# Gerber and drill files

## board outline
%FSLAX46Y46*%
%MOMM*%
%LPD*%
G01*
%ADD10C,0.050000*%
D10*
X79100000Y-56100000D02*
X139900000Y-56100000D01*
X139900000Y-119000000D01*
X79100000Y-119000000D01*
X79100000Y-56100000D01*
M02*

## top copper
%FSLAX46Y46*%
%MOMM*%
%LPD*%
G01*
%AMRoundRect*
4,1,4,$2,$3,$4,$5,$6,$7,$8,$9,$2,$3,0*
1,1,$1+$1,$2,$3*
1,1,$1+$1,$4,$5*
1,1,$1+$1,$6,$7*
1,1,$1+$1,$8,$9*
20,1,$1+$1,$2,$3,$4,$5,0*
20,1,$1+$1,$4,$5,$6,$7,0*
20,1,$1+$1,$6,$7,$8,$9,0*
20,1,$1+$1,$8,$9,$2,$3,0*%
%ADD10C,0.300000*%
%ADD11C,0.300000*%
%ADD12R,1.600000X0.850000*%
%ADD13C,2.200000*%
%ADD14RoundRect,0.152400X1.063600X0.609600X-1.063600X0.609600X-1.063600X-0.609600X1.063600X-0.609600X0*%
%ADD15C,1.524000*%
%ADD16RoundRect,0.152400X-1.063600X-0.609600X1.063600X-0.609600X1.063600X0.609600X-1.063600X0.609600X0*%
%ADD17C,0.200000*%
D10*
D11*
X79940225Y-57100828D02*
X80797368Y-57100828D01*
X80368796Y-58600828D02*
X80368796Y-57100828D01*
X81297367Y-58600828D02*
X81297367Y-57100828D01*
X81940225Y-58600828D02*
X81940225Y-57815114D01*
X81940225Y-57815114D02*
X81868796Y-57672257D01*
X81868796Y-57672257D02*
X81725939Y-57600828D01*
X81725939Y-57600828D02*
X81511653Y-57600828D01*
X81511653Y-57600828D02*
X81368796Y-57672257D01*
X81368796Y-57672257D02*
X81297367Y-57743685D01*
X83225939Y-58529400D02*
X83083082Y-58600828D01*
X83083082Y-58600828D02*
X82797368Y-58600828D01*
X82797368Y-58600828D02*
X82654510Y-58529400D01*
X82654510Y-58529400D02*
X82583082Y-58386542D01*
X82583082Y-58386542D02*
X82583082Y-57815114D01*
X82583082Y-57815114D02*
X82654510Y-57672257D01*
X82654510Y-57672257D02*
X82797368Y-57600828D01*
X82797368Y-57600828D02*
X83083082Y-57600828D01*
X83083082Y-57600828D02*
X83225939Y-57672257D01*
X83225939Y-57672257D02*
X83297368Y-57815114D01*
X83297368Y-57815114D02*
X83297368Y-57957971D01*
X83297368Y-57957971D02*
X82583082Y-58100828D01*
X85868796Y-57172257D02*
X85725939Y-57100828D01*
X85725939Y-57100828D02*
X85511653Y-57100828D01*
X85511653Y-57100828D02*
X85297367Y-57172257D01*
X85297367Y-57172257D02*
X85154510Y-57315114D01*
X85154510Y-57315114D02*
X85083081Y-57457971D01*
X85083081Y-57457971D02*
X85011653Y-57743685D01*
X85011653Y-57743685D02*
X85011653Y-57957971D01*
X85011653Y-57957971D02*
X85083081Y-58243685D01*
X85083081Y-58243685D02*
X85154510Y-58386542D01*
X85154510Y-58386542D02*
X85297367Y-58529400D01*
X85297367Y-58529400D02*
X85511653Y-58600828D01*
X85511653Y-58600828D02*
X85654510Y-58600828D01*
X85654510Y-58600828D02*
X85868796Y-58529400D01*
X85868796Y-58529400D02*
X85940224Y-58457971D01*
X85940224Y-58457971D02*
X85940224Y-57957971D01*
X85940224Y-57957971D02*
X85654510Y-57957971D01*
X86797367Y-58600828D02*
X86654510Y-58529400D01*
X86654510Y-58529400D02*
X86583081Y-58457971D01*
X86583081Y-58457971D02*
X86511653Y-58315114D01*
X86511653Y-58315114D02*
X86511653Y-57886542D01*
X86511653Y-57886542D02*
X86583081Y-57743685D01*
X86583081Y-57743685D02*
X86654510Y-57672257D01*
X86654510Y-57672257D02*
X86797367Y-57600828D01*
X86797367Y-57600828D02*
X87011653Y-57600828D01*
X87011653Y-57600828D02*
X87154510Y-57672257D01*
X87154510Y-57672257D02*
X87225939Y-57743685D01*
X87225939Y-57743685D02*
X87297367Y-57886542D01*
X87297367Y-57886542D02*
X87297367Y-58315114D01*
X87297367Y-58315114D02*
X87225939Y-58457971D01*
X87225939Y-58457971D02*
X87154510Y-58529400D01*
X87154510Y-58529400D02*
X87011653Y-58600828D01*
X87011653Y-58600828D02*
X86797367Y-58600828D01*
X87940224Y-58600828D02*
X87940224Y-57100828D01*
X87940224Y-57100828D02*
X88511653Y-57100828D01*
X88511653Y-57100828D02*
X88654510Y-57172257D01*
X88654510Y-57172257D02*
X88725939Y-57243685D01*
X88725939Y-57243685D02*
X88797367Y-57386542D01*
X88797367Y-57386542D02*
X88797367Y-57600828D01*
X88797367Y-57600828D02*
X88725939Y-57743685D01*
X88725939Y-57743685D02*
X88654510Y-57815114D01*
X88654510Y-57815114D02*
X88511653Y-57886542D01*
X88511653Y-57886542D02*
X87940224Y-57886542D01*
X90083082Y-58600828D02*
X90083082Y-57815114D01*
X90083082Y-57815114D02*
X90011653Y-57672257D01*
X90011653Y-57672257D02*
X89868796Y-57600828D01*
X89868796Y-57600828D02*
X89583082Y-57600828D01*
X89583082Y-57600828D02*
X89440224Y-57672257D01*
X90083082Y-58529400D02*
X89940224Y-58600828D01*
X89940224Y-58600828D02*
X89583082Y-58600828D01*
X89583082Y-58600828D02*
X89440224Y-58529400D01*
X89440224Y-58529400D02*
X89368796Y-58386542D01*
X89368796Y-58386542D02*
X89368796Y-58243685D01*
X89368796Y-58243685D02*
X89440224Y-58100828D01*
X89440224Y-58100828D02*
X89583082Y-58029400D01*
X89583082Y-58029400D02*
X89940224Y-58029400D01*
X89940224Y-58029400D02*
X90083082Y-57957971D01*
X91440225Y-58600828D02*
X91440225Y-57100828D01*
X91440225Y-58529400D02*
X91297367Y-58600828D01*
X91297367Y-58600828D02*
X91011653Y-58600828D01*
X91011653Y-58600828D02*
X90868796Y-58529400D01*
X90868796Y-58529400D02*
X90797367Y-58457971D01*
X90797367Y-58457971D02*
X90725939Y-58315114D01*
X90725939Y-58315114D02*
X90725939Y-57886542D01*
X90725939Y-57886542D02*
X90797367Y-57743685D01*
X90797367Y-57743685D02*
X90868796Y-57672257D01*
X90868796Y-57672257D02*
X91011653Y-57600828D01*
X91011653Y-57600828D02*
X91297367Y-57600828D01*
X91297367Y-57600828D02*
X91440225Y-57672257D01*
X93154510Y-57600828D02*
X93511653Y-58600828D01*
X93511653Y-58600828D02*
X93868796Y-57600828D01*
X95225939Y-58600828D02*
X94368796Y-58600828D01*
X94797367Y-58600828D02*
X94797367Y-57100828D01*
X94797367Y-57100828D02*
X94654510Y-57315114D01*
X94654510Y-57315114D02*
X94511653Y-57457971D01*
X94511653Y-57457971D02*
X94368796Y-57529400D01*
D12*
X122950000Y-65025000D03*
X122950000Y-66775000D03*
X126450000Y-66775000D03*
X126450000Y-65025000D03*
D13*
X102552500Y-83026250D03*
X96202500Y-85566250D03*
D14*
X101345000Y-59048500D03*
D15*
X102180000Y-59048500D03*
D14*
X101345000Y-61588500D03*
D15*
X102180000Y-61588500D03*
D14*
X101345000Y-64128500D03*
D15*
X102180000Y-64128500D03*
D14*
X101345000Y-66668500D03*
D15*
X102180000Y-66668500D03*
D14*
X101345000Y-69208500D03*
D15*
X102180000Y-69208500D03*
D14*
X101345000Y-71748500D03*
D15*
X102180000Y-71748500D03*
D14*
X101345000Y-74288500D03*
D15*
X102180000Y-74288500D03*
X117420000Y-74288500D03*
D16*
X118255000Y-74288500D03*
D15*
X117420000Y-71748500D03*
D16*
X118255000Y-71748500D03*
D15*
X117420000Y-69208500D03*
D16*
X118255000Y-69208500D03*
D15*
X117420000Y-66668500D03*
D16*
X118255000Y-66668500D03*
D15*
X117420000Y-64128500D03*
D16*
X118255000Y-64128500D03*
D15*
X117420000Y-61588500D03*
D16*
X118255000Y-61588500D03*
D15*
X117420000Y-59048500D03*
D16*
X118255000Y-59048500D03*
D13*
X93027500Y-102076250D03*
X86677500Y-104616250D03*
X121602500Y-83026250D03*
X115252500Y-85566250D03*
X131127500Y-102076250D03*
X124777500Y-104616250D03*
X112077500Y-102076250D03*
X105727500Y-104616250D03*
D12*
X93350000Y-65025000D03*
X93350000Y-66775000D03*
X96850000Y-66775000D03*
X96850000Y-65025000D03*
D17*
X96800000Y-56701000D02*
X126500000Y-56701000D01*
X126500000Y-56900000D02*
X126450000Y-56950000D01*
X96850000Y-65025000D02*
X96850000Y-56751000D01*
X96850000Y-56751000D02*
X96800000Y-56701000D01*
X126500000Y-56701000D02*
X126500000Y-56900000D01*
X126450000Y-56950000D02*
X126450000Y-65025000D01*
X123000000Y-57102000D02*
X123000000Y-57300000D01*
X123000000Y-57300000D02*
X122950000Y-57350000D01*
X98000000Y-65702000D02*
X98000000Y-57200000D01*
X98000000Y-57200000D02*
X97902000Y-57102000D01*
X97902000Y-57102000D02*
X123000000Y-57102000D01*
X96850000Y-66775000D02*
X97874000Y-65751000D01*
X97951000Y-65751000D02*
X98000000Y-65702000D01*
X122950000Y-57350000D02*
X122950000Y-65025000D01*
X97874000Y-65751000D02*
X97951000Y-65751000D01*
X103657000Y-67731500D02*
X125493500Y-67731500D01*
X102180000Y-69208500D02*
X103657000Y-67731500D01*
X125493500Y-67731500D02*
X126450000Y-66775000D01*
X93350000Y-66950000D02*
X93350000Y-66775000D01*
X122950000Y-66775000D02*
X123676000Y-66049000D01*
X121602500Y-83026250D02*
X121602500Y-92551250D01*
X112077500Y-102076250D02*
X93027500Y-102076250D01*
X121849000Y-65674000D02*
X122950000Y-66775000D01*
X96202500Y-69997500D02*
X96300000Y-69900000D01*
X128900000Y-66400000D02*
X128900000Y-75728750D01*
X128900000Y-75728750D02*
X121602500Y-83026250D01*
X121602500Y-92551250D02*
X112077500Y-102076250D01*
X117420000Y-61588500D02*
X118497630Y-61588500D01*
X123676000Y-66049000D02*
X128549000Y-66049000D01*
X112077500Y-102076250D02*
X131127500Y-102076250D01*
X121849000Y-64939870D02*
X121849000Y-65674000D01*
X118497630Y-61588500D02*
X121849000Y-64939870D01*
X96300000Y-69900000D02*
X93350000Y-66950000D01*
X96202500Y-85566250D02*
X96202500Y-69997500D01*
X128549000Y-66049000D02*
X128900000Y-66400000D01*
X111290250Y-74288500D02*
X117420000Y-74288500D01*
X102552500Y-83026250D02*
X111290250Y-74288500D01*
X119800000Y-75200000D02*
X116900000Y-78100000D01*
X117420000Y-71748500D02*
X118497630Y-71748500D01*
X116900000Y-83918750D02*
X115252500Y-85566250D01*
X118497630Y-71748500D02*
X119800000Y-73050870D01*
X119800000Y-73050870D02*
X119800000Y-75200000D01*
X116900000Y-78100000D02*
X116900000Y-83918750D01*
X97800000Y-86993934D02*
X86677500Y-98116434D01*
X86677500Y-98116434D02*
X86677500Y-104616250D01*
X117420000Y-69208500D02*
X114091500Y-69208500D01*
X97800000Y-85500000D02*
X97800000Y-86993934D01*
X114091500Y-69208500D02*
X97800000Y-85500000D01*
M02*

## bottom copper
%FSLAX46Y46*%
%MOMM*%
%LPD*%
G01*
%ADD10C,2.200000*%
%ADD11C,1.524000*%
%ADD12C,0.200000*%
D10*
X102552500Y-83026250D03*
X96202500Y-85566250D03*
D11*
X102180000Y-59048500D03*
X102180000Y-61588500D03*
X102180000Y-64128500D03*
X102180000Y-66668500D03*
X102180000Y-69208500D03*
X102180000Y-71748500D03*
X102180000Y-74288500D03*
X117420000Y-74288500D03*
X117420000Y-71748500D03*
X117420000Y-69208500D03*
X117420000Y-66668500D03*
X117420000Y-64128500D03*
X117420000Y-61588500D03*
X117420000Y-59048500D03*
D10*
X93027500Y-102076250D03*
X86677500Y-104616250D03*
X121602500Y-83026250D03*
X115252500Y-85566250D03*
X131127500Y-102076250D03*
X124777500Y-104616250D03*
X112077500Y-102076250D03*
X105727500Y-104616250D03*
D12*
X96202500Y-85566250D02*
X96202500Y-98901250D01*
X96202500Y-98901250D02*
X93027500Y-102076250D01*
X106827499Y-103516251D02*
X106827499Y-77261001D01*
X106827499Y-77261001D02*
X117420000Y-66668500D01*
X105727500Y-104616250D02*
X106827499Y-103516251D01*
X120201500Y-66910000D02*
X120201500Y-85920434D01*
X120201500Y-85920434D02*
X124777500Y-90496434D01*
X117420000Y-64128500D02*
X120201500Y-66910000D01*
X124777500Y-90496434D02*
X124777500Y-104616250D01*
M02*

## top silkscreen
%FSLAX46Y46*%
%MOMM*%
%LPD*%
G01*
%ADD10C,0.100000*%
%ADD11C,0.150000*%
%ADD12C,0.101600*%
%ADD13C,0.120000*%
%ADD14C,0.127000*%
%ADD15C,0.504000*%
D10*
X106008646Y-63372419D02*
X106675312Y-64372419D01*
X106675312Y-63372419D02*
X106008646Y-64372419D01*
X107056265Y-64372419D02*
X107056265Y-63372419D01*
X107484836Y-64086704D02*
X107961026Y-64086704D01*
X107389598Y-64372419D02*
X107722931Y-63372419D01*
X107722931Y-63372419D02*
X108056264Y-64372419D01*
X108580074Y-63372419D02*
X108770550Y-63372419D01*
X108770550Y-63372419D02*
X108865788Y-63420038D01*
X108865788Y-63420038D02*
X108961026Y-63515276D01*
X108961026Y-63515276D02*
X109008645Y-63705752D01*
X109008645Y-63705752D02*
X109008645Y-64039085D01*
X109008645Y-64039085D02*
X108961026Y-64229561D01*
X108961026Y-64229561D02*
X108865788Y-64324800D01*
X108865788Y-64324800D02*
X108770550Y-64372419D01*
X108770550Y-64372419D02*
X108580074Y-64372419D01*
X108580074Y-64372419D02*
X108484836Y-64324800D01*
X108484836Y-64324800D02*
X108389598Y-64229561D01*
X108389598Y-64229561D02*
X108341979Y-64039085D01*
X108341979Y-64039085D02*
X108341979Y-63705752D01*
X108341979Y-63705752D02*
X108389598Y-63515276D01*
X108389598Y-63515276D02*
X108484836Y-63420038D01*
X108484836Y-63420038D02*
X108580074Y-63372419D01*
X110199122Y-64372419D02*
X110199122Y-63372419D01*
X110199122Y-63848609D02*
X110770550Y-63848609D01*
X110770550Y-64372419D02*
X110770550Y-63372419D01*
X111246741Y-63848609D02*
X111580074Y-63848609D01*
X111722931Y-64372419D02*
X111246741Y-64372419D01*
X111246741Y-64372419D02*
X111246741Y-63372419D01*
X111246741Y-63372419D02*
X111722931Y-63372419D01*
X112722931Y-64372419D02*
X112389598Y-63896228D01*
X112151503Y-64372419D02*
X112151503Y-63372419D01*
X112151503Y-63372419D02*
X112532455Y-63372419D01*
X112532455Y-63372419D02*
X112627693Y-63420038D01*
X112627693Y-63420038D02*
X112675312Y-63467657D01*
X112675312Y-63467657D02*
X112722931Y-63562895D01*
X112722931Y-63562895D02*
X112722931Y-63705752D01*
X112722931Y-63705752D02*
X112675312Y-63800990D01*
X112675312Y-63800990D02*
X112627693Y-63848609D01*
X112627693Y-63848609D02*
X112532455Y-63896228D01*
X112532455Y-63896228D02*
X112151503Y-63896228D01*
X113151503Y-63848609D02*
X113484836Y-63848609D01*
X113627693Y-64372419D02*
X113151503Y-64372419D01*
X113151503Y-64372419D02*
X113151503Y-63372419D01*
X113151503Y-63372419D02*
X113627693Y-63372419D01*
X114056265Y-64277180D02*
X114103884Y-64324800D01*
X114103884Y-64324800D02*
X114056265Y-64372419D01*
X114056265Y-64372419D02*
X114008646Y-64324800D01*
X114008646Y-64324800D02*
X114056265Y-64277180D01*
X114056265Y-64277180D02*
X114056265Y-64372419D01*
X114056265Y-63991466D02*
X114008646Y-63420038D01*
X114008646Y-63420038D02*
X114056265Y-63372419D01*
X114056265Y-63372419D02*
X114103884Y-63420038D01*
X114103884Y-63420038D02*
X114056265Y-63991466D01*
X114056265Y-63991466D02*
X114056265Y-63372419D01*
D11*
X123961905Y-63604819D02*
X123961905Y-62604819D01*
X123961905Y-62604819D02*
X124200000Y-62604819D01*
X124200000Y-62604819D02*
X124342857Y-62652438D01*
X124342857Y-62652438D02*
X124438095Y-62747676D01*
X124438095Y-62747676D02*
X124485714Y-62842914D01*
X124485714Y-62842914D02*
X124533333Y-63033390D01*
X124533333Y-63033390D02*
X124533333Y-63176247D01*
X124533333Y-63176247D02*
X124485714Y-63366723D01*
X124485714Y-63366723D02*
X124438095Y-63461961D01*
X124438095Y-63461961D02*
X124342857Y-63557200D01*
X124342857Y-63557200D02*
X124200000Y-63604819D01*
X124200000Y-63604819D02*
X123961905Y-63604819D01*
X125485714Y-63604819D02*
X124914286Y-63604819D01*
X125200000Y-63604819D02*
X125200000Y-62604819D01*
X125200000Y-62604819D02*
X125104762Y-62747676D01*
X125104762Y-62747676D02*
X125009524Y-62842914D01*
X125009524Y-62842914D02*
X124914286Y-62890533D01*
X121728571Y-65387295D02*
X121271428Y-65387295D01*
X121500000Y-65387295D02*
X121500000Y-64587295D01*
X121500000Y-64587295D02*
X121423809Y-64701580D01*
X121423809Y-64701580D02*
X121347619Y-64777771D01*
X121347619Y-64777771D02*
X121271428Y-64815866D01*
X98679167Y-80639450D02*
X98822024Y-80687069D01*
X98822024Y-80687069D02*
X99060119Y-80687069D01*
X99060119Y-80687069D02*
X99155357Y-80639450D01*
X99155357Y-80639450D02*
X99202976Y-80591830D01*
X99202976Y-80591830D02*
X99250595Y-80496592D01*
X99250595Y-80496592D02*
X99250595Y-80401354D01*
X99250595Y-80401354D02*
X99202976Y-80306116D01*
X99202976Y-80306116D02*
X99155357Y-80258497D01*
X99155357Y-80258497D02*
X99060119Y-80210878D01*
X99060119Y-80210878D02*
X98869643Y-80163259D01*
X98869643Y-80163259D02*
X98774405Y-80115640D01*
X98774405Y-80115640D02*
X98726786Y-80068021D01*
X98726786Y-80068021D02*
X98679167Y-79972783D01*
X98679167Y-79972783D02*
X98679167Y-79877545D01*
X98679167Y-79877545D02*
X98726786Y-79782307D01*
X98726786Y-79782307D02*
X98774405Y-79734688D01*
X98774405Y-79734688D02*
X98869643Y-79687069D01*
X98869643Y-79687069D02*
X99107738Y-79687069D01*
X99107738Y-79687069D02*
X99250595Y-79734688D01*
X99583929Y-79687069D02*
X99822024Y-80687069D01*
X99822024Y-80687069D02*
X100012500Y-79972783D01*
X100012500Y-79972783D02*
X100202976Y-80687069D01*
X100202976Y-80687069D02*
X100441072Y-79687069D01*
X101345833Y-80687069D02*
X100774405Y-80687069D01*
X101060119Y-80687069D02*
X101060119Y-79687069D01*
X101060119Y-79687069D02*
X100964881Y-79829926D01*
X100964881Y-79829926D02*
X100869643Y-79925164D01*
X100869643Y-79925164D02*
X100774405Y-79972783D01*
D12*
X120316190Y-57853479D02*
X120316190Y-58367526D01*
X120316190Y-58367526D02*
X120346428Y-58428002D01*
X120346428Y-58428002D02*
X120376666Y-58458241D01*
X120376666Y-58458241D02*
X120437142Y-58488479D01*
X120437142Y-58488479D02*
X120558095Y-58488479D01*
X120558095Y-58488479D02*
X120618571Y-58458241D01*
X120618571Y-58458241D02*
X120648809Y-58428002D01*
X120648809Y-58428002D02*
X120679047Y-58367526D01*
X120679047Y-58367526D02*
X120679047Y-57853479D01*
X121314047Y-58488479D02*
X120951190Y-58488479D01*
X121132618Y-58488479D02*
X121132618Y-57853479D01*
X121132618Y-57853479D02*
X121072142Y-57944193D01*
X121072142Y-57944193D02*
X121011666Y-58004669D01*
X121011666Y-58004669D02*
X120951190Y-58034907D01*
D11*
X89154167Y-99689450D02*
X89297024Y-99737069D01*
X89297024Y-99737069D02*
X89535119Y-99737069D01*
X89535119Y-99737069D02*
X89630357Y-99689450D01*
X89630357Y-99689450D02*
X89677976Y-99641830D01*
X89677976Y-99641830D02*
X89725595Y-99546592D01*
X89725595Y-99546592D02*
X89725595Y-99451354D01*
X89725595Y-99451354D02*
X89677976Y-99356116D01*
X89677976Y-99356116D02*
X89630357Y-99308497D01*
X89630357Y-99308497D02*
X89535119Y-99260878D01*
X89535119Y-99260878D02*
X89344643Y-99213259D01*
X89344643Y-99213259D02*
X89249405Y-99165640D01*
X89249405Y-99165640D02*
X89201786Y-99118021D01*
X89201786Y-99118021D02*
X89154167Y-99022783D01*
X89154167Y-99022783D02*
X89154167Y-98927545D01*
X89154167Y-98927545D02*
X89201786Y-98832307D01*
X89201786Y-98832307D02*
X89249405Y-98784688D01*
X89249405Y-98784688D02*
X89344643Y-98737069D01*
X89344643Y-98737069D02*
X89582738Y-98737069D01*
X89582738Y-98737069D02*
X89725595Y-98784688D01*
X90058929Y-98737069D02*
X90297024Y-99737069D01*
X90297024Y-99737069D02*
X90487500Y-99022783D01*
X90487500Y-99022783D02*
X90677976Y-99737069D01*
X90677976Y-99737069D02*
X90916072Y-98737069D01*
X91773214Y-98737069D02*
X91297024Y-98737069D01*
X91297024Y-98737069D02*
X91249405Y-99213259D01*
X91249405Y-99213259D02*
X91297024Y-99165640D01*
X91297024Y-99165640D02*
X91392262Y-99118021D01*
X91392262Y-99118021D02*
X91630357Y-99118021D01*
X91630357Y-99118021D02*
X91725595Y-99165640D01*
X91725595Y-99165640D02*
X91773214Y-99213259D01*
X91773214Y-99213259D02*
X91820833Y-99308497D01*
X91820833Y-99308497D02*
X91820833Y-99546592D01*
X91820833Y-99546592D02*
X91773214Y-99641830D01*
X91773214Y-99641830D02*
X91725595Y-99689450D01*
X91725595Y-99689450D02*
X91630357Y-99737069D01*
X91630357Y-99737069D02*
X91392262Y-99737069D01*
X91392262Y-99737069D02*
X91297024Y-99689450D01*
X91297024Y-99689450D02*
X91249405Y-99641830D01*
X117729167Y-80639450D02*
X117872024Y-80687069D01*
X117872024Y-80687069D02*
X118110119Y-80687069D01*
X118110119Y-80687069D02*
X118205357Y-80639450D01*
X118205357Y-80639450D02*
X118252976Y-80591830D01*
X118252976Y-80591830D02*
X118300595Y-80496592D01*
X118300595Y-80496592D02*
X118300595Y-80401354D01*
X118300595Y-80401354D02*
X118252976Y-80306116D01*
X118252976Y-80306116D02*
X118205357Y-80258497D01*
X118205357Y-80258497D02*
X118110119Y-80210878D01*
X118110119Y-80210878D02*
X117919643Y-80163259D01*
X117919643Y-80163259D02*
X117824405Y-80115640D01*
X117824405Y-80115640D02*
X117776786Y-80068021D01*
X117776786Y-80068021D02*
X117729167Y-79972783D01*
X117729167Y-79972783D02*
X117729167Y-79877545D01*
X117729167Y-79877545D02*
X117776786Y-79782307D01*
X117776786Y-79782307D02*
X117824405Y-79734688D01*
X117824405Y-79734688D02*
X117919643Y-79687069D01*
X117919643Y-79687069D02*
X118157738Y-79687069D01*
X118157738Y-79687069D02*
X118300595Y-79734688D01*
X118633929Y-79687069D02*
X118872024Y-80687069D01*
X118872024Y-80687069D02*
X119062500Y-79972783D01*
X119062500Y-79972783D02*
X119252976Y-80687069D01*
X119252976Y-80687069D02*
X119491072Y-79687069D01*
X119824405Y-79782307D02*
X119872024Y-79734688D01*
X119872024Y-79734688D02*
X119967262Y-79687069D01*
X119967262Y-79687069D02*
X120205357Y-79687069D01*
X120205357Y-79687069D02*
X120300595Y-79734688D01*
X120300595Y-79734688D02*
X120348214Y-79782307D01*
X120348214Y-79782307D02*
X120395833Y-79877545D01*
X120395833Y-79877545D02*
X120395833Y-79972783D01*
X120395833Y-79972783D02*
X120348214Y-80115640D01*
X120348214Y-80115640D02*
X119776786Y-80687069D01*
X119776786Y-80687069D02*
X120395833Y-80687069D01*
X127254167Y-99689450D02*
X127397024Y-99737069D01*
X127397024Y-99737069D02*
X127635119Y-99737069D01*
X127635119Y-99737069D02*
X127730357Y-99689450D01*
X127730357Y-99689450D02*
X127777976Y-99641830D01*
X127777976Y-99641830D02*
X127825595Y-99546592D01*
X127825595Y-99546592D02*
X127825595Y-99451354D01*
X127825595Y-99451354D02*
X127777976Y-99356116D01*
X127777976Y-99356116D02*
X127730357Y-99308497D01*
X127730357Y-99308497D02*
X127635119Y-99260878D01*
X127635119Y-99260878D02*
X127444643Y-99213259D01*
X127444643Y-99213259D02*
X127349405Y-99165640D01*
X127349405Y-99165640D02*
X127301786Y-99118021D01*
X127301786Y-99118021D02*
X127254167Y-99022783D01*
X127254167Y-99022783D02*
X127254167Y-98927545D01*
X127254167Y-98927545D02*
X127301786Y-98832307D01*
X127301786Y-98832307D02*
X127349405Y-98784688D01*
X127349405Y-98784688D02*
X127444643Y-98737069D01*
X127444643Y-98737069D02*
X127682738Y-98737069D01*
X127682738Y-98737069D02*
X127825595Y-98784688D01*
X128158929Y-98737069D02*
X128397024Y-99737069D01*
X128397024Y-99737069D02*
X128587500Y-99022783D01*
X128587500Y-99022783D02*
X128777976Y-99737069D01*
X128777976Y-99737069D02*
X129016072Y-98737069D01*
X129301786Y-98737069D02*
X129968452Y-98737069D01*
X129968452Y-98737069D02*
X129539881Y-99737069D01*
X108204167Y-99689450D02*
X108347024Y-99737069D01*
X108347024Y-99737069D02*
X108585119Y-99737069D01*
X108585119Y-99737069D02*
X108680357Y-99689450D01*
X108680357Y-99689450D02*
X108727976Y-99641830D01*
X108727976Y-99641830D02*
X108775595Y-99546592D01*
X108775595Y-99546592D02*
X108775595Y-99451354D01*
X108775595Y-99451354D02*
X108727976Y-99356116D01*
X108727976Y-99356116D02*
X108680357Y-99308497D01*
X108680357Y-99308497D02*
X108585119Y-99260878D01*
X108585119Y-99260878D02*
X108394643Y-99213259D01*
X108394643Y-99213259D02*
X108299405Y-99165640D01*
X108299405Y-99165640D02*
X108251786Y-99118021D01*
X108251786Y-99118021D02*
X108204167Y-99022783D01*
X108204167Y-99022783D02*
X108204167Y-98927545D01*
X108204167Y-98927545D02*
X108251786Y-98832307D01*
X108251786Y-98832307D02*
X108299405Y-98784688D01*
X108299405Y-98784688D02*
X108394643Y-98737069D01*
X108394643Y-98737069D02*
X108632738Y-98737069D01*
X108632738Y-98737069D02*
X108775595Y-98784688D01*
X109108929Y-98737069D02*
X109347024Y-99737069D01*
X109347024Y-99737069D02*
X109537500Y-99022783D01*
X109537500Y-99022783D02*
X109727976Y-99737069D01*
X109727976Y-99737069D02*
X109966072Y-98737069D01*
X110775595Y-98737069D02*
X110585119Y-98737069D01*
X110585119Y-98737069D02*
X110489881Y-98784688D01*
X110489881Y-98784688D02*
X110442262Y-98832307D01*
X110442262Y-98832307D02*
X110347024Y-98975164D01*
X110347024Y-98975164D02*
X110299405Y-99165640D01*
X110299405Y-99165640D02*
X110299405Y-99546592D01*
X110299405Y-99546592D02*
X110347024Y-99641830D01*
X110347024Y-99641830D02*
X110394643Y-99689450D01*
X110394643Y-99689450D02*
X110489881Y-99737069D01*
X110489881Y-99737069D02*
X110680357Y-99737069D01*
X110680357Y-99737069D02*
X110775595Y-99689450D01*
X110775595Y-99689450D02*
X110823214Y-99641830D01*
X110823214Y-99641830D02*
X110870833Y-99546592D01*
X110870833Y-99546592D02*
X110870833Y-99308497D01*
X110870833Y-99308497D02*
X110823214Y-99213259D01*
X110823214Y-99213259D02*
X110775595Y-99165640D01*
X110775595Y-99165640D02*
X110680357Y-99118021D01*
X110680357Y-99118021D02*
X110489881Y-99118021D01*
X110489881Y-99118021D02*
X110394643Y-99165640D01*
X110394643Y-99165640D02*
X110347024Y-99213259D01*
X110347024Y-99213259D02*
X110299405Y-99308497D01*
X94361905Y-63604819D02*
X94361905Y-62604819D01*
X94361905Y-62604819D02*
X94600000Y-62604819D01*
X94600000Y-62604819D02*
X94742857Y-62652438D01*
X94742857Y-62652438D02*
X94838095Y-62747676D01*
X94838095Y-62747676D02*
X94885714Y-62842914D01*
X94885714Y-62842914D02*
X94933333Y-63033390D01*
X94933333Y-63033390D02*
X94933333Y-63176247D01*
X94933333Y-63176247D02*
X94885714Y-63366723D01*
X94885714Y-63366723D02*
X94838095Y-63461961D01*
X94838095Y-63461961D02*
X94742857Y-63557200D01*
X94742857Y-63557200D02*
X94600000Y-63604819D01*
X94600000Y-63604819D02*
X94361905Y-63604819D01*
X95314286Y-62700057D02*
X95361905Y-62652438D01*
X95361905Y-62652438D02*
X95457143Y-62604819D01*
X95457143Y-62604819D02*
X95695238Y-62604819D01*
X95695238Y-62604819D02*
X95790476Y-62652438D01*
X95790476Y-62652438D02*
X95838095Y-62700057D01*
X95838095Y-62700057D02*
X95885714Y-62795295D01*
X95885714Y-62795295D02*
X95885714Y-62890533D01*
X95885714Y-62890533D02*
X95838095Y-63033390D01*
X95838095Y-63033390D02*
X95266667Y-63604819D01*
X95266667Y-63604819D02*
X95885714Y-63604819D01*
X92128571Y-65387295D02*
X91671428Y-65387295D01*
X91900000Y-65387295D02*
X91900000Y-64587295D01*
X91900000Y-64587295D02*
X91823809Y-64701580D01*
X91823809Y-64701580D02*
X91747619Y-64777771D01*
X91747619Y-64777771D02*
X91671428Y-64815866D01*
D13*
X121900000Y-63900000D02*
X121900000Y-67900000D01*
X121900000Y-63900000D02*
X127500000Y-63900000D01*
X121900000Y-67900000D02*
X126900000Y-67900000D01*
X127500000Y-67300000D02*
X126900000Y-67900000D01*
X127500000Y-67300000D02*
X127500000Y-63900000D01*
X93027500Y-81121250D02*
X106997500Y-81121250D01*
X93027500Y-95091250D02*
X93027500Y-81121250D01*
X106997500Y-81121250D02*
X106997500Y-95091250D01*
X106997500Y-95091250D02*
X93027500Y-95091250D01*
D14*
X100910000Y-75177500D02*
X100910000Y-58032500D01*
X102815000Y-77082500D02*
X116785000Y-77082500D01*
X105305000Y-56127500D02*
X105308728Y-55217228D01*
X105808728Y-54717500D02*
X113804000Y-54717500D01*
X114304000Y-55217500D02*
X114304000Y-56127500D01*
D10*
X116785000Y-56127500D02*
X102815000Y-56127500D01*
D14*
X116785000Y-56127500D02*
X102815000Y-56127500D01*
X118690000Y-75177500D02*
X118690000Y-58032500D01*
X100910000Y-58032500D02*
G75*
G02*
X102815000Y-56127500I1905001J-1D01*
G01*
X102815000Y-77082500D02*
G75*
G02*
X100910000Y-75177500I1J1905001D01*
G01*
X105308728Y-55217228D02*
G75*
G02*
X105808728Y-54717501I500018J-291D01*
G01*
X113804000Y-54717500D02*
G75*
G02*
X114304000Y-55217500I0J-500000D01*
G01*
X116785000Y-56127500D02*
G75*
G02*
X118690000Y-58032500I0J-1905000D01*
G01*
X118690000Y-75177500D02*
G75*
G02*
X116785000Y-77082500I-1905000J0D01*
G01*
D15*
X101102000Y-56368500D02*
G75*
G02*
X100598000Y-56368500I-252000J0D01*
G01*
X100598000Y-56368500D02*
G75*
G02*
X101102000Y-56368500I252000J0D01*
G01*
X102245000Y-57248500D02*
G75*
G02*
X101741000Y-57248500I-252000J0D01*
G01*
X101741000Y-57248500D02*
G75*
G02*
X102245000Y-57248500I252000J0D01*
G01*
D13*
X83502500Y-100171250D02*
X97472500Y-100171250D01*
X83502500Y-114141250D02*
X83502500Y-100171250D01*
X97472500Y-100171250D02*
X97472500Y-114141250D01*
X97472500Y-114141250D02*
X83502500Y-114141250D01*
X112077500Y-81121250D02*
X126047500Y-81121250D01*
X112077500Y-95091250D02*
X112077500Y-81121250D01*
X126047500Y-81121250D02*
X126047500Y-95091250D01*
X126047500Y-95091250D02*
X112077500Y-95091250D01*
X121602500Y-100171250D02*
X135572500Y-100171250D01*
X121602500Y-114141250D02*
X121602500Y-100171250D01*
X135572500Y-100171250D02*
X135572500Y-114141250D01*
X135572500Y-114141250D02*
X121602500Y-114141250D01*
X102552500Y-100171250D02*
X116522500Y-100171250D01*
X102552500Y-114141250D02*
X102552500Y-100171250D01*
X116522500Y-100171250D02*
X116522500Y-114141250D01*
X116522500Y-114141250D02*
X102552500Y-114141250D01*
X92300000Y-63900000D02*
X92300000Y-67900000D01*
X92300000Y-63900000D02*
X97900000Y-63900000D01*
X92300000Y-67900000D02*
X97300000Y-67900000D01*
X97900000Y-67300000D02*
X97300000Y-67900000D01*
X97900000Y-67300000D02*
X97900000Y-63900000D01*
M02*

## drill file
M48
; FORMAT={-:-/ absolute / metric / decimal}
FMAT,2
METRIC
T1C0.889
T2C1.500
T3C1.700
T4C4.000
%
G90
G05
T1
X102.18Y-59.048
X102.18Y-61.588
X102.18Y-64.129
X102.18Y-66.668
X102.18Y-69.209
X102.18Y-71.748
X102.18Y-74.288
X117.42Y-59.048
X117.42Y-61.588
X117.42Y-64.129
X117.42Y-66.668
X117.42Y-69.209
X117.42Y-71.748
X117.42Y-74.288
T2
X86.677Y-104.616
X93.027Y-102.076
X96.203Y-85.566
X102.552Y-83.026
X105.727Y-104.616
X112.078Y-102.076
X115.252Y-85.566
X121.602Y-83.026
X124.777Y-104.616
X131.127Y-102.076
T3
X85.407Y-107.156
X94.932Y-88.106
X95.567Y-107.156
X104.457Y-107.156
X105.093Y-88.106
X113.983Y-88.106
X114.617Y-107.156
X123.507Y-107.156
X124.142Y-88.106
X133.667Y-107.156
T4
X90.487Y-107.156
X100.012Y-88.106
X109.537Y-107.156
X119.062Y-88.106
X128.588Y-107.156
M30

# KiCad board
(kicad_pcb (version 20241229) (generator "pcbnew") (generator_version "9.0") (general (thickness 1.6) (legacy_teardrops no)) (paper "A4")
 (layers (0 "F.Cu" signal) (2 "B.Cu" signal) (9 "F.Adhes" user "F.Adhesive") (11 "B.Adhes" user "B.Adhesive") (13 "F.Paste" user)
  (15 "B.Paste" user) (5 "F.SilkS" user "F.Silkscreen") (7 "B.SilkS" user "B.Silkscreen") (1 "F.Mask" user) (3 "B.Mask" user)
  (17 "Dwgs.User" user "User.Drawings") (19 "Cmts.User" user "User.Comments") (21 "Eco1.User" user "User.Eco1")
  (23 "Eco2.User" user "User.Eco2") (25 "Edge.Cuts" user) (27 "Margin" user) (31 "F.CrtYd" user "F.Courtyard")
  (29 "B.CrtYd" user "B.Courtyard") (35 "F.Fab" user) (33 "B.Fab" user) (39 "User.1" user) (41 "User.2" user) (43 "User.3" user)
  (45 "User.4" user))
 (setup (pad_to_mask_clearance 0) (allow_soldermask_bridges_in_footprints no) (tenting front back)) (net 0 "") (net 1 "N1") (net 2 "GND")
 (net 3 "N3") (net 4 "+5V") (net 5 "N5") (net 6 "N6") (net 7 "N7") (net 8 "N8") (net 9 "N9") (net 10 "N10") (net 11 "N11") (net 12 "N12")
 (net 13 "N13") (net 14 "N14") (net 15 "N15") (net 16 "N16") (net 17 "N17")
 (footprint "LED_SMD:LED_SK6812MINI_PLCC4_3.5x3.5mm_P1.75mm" (layer "F.Cu") (at 124.7 65.9)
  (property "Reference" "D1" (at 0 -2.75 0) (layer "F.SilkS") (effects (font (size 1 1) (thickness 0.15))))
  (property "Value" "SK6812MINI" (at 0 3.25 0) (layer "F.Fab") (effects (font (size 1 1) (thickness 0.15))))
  (fp_line (start -2.8 -2) (end -2.8 2) (stroke (width 0.12) (type default)) (layer "F.SilkS"))
  (fp_line (start -2.8 -2) (end 2.8 -2) (stroke (width 0.12) (type solid)) (layer "F.SilkS"))
  (fp_line (start -2.8 2) (end 2.2 2) (stroke (width 0.12) (type solid)) (layer "F.SilkS"))
  (fp_line (start 2.8 1.4) (end 2.2 2) (stroke (width 0.12) (type default)) (layer "F.SilkS"))
  (fp_line (start 2.8 1.4) (end 2.8 -2) (stroke (width 0.12) (type solid)) (layer "F.SilkS"))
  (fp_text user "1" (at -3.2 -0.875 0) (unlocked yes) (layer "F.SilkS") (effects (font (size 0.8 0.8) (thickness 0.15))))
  (pad "1" smd rect (at -1.75 -0.875) (size 1.6 0.85) (layers "F.Cu" "F.Mask" "F.Paste") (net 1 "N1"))
  (pad "2" smd rect (at -1.75 0.875) (size 1.6 0.85) (layers "F.Cu" "F.Mask" "F.Paste") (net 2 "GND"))
  (pad "3" smd rect (at 1.75 0.875) (size 1.6 0.85) (layers "F.Cu" "F.Mask" "F.Paste") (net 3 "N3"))
  (pad "4" smd rect (at 1.75 -0.875) (size 1.6 0.85) (layers "F.Cu" "F.Mask" "F.Paste") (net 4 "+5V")))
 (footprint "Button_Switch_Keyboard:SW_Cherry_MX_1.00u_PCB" (layer "F.Cu") (at 102.5525 83.02625)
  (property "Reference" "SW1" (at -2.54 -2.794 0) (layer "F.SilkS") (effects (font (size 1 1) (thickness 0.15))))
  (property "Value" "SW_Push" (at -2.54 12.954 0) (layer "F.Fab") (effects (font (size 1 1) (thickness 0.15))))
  (fp_line (start -9.525 -1.905) (end 4.445 -1.905) (stroke (width 0.12) (type solid)) (layer "F.SilkS"))
  (fp_line (start -9.525 12.065) (end -9.525 -1.905) (stroke (width 0.12) (type solid)) (layer "F.SilkS"))
  (fp_line (start 4.445 -1.905) (end 4.445 12.065) (stroke (width 0.12) (type solid)) (layer "F.SilkS"))
  (fp_line (start 4.445 12.065) (end -9.525 12.065) (stroke (width 0.12) (type solid)) (layer "F.SilkS"))
  (pad "" np_thru_hole circle (at -7.62 5.08) (size 1.7 1.7) (drill 1.7) (layers "*.Cu" "*.Mask"))
  (pad "" np_thru_hole circle (at -2.54 5.08) (size 4 4) (drill 4) (layers "*.Cu" "*.Mask"))
  (pad "" np_thru_hole circle (at 2.54 5.08) (size 1.7 1.7) (drill 1.7) (layers "*.Cu" "*.Mask"))
  (pad "1" thru_hole circle (at 0 0) (size 2.2 2.2) (drill 1.5) (layers "*.Cu" "*.Mask") (remove_unused_layers no) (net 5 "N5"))
  (pad "2" thru_hole circle (at -6.35 2.54) (size 2.2 2.2) (drill 1.5) (layers "*.Cu" "*.Mask") (remove_unused_layers no) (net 2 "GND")))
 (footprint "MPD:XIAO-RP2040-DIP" (layer "F.Cu") (at 109.8 66.6685)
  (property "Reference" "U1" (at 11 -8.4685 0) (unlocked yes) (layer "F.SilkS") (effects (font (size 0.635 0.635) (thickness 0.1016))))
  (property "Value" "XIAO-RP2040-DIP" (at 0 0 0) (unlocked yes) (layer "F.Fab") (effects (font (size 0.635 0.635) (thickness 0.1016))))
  (fp_line (start -8.89 8.509) (end -8.89 -8.636) (stroke (width 0.127) (type solid)) (layer "F.SilkS"))
  (fp_line (start -6.985 10.414) (end 6.985 10.414) (stroke (width 0.127) (type solid)) (layer "F.SilkS"))
  (fp_line (start -4.495 -10.541) (end -4.491272 -11.451272) (stroke (width 0.127) (type solid)) (layer "F.SilkS"))
  (fp_line (start -3.991272 -11.951) (end 4.004 -11.951) (stroke (width 0.127) (type solid)) (layer "F.SilkS"))
  (fp_line (start 4.504 -11.451) (end 4.504 -10.541) (stroke (width 0.127) (type solid)) (layer "F.SilkS"))
  (fp_line (start 6.985 -10.541) (end -6.985 -10.541) (stroke (width 0.1) (type solid)) (layer "F.SilkS"))
  (fp_line (start 6.985 -10.541) (end -6.985 -10.541) (stroke (width 0.127) (type solid)) (layer "F.SilkS"))
  (fp_line (start 8.89 8.509) (end 8.89 -8.636) (stroke (width 0.127) (type solid)) (layer "F.SilkS"))
  (fp_arc (start -8.89 -8.636) (mid -8.332038 -9.983038) (end -6.985 -10.541) (stroke (width 0.127) (type solid)) (layer "F.SilkS"))
  (fp_arc (start -6.985 10.414) (mid -8.332038 9.856038) (end -8.89 8.509) (stroke (width 0.127) (type solid)) (layer "F.SilkS"))
  (fp_arc (start -4.491272 -11.451272) (mid -4.344728 -11.80464) (end -3.991272 -11.951) (stroke (width 0.127) (type default))
   (layer "F.SilkS"))
  (fp_arc (start 4.004 -11.951) (mid 4.357553 -11.804553) (end 4.504 -11.451) (stroke (width 0.127) (type default)) (layer "F.SilkS"))
  (fp_arc (start 6.985 -10.541) (mid 8.332038 -9.983038) (end 8.89 -8.636) (stroke (width 0.127) (type solid)) (layer "F.SilkS"))
  (fp_arc (start 8.89 8.509) (mid 8.332038 9.856038) (end 6.985 10.414) (stroke (width 0.127) (type solid)) (layer "F.SilkS"))
  (fp_circle (center -8.95 -10.3) (end -8.95 -10.554) (stroke (width 0.5) (type solid)) (fill yes) (layer "F.SilkS"))
  (fp_circle (center -7.807 -9.42) (end -7.807 -9.674) (stroke (width 0.5) (type solid)) (fill yes) (layer "F.SilkS"))
  (pad "1" smd roundrect (at -8.455 -7.62 180) (size 2.432 1.524) (layers "F.Cu" "F.Mask") (roundrect_rratio 0.1) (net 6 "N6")
   (thermal_bridge_angle 45))
  (pad "1" thru_hole circle (at -7.62 -7.62 180) (size 1.524 1.524) (drill 0.889) (layers "*.Cu" "*.Mask") (remove_unused_layers no)
   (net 6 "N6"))
  (pad "2" smd roundrect (at -8.455 -5.08 180) (size 2.432 1.524) (layers "F.Cu" "F.Mask") (roundrect_rratio 0.1) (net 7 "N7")
   (thermal_bridge_angle 45))
  (pad "2" thru_hole circle (at -7.62 -5.08 180) (size 1.524 1.524) (drill 0.889) (layers "*.Cu" "*.Mask") (remove_unused_layers no)
   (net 7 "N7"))
  (pad "3" smd roundrect (at -8.455 -2.54 180) (size 2.432 1.524) (layers "F.Cu" "F.Mask") (roundrect_rratio 0.1) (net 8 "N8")
   (thermal_bridge_angle 45))
  (pad "3" thru_hole circle (at -7.62 -2.54 180) (size 1.524 1.524) (drill 0.889) (layers "*.Cu" "*.Mask") (remove_unused_layers no)
   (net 8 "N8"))
  (pad "4" smd roundrect (at -8.455 0 180) (size 2.432 1.524) (layers "F.Cu" "F.Mask") (roundrect_rratio 0.1) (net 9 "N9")
   (thermal_bridge_angle 45))
  (pad "4" thru_hole circle (at -7.62 0 180) (size 1.524 1.524) (drill 0.889) (layers "*.Cu" "*.Mask") (remove_unused_layers no)
   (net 9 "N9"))
  (pad "5" smd roundrect (at -8.455 2.54 180) (size 2.432 1.524) (layers "F.Cu" "F.Mask") (roundrect_rratio 0.1) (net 3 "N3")
   (thermal_bridge_angle 45))
  (pad "5" thru_hole circle (at -7.62 2.54 180) (size 1.524 1.524) (drill 0.889) (layers "*.Cu" "*.Mask") (remove_unused_layers no)
   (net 3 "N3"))
  (pad "6" smd roundrect (at -8.455 5.08 180) (size 2.432 1.524) (layers "F.Cu" "F.Mask") (roundrect_rratio 0.1) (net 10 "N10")
   (thermal_bridge_angle 45))
  (pad "6" thru_hole circle (at -7.62 5.08 180) (size 1.524 1.524) (drill 0.889) (layers "*.Cu" "*.Mask") (remove_unused_layers no)
   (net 10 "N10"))
  (pad "7" smd roundrect (at -8.455 7.62 180) (size 2.432 1.524) (layers "F.Cu" "F.Mask") (roundrect_rratio 0.1) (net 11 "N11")
   (thermal_bridge_angle 45))
  (pad "7" thru_hole circle (at -7.62 7.62 180) (size 1.524 1.524) (drill 0.889) (layers "*.Cu" "*.Mask") (remove_unused_layers no)
   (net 11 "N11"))
  (pad "8" thru_hole circle (at 7.62 7.62) (size 1.524 1.524) (drill 0.889) (layers "*.Cu" "*.Mask") (remove_unused_layers no) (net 5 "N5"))
  (pad "8" smd roundrect (at 8.455 7.62) (size 2.432 1.524) (layers "F.Cu" "F.Mask") (roundrect_rratio 0.1) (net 5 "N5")
   (thermal_bridge_angle 45))
  (pad "9" thru_hole circle (at 7.62 5.08) (size 1.524 1.524) (drill 0.889) (layers "*.Cu" "*.Mask") (remove_unused_layers no)
   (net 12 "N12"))
  (pad "9" smd roundrect (at 8.455 5.08) (size 2.432 1.524) (layers "F.Cu" "F.Mask") (roundrect_rratio 0.1) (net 12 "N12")
   (thermal_bridge_angle 45))
  (pad "10" thru_hole circle (at 7.62 2.54) (size 1.524 1.524) (drill 0.889) (layers "*.Cu" "*.Mask") (remove_unused_layers no)
   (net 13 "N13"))
  (pad "10" smd roundrect (at 8.455 2.54) (size 2.432 1.524) (layers "F.Cu" "F.Mask") (roundrect_rratio 0.1) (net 13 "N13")
   (thermal_bridge_angle 45))
  (pad "11" thru_hole circle (at 7.62 0) (size 1.524 1.524) (drill 0.889) (layers "*.Cu" "*.Mask") (remove_unused_layers no) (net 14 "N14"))
  (pad "11" smd roundrect (at 8.455 0) (size 2.432 1.524) (layers "F.Cu" "F.Mask") (roundrect_rratio 0.1) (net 14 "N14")
   (thermal_bridge_angle 45))
  (pad "12" thru_hole circle (at 7.62 -2.54) (size 1.524 1.524) (drill 0.889) (layers "*.Cu" "*.Mask") (remove_unused_layers no)
   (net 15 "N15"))
  (pad "12" smd roundrect (at 8.455 -2.54) (size 2.432 1.524) (layers "F.Cu" "F.Mask") (roundrect_rratio 0.1) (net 15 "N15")
   (thermal_bridge_angle 45))
  (pad "13" thru_hole circle (at 7.62 -5.08) (size 1.524 1.524) (drill 0.889) (layers "*.Cu" "*.Mask") (remove_unused_layers no)
   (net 2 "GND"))
  (pad "13" smd roundrect (at 8.455 -5.08) (size 2.432 1.524) (layers "F.Cu" "F.Mask") (roundrect_rratio 0.1) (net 2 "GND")
   (thermal_bridge_angle 45))
  (pad "14" thru_hole circle (at 7.62 -7.62) (size 1.524 1.524) (drill 0.889) (layers "*.Cu" "*.Mask") (remove_unused_layers no)
   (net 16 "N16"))
  (pad "14" smd roundrect (at 8.455 -7.62) (size 2.432 1.524) (layers "F.Cu" "F.Mask") (roundrect_rratio 0.1) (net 16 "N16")
   (thermal_bridge_angle 45)))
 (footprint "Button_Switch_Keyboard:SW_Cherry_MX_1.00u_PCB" (layer "F.Cu") (at 93.0275 102.07625)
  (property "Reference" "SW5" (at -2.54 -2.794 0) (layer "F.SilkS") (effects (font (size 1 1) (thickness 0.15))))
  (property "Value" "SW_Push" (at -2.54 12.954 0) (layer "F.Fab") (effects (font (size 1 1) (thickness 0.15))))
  (fp_line (start -9.525 -1.905) (end 4.445 -1.905) (stroke (width 0.12) (type solid)) (layer "F.SilkS"))
  (fp_line (start -9.525 12.065) (end -9.525 -1.905) (stroke (width 0.12) (type solid)) (layer "F.SilkS"))
  (fp_line (start 4.445 -1.905) (end 4.445 12.065) (stroke (width 0.12) (type solid)) (layer "F.SilkS"))
  (fp_line (start 4.445 12.065) (end -9.525 12.065) (stroke (width 0.12) (type solid)) (layer "F.SilkS"))
  (pad "" np_thru_hole circle (at -7.62 5.08) (size 1.7 1.7) (drill 1.7) (layers "*.Cu" "*.Mask"))
  (pad "" np_thru_hole circle (at -2.54 5.08) (size 4 4) (drill 4) (layers "*.Cu" "*.Mask"))
  (pad "" np_thru_hole circle (at 2.54 5.08) (size 1.7 1.7) (drill 1.7) (layers "*.Cu" "*.Mask"))
  (pad "1" thru_hole circle (at 0 0) (size 2.2 2.2) (drill 1.5) (layers "*.Cu" "*.Mask") (remove_unused_layers no) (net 2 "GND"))
  (pad "2" thru_hole circle (at -6.35 2.54) (size 2.2 2.2) (drill 1.5) (layers "*.Cu" "*.Mask") (remove_unused_layers no) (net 13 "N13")))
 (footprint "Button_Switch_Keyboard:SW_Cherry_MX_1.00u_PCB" (layer "F.Cu") (at 121.6025 83.02625)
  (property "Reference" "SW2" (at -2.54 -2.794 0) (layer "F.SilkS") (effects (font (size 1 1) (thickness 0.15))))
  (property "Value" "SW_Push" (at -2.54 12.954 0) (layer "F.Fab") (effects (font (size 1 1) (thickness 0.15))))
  (fp_line (start -9.525 -1.905) (end 4.445 -1.905) (stroke (width 0.12) (type solid)) (layer "F.SilkS"))
  (fp_line (start -9.525 12.065) (end -9.525 -1.905) (stroke (width 0.12) (type solid)) (layer "F.SilkS"))
  (fp_line (start 4.445 -1.905) (end 4.445 12.065) (stroke (width 0.12) (type solid)) (layer "F.SilkS"))
  (fp_line (start 4.445 12.065) (end -9.525 12.065) (stroke (width 0.12) (type solid)) (layer "F.SilkS"))
  (pad "" np_thru_hole circle (at -7.62 5.08) (size 1.7 1.7) (drill 1.7) (layers "*.Cu" "*.Mask"))
  (pad "" np_thru_hole circle (at -2.54 5.08) (size 4 4) (drill 4) (layers "*.Cu" "*.Mask"))
  (pad "" np_thru_hole circle (at 2.54 5.08) (size 1.7 1.7) (drill 1.7) (layers "*.Cu" "*.Mask"))
  (pad "1" thru_hole circle (at 0 0) (size 2.2 2.2) (drill 1.5) (layers "*.Cu" "*.Mask") (remove_unused_layers no) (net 2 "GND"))
  (pad "2" thru_hole circle (at -6.35 2.54) (size 2.2 2.2) (drill 1.5) (layers "*.Cu" "*.Mask") (remove_unused_layers no) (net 12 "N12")))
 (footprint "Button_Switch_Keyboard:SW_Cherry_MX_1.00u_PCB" (layer "F.Cu") (at 131.1275 102.07625)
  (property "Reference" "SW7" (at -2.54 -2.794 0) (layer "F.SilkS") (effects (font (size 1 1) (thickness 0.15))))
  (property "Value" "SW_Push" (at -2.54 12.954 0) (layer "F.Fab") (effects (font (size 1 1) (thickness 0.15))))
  (fp_line (start -9.525 -1.905) (end 4.445 -1.905) (stroke (width 0.12) (type solid)) (layer "F.SilkS"))
  (fp_line (start -9.525 12.065) (end -9.525 -1.905) (stroke (width 0.12) (type solid)) (layer "F.SilkS"))
  (fp_line (start 4.445 -1.905) (end 4.445 12.065) (stroke (width 0.12) (type solid)) (layer "F.SilkS"))
  (fp_line (start 4.445 12.065) (end -9.525 12.065) (stroke (width 0.12) (type solid)) (layer "F.SilkS"))
  (pad "" np_thru_hole circle (at -7.62 5.08) (size 1.7 1.7) (drill 1.7) (layers "*.Cu" "*.Mask"))
  (pad "" np_thru_hole circle (at -2.54 5.08) (size 4 4) (drill 4) (layers "*.Cu" "*.Mask"))
  (pad "" np_thru_hole circle (at 2.54 5.08) (size 1.7 1.7) (drill 1.7) (layers "*.Cu" "*.Mask"))
  (pad "1" thru_hole circle (at 0 0) (size 2.2 2.2) (drill 1.5) (layers "*.Cu" "*.Mask") (remove_unused_layers no) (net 2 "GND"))
  (pad "2" thru_hole circle (at -6.35 2.54) (size 2.2 2.2) (drill 1.5) (layers "*.Cu" "*.Mask") (remove_unused_layers no) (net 15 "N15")))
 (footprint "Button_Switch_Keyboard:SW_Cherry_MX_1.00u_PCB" (layer "F.Cu") (at 112.0775 102.07625)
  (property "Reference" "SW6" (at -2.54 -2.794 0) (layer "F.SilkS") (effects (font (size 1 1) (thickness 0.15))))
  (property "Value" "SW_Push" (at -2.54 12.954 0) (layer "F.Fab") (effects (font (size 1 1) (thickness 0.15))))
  (fp_line (start -9.525 -1.905) (end 4.445 -1.905) (stroke (width 0.12) (type solid)) (layer "F.SilkS"))
  (fp_line (start -9.525 12.065) (end -9.525 -1.905) (stroke (width 0.12) (type solid)) (layer "F.SilkS"))
  (fp_line (start 4.445 -1.905) (end 4.445 12.065) (stroke (width 0.12) (type solid)) (layer "F.SilkS"))
  (fp_line (start 4.445 12.065) (end -9.525 12.065) (stroke (width 0.12) (type solid)) (layer "F.SilkS"))
  (pad "" np_thru_hole circle (at -7.62 5.08) (size 1.7 1.7) (drill 1.7) (layers "*.Cu" "*.Mask"))
  (pad "" np_thru_hole circle (at -2.54 5.08) (size 4 4) (drill 4) (layers "*.Cu" "*.Mask"))
  (pad "" np_thru_hole circle (at 2.54 5.08) (size 1.7 1.7) (drill 1.7) (layers "*.Cu" "*.Mask"))
  (pad "1" thru_hole circle (at 0 0) (size 2.2 2.2) (drill 1.5) (layers "*.Cu" "*.Mask") (remove_unused_layers no) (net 2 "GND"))
  (pad "2" thru_hole circle (at -6.35 2.54) (size 2.2 2.2) (drill 1.5) (layers "*.Cu" "*.Mask") (remove_unused_layers no) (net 14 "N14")))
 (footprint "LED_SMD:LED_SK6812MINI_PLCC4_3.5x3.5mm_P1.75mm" (layer "F.Cu") (at 95.1 65.9)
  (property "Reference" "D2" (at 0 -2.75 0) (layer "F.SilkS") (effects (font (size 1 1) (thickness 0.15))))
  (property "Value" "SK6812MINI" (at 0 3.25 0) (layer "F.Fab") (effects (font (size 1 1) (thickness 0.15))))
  (fp_line (start -2.8 -2) (end -2.8 2) (stroke (width 0.12) (type default)) (layer "F.SilkS"))
  (fp_line (start -2.8 -2) (end 2.8 -2) (stroke (width 0.12) (type solid)) (layer "F.SilkS"))
  (fp_line (start -2.8 2) (end 2.2 2) (stroke (width 0.12) (type solid)) (layer "F.SilkS"))
  (fp_line (start 2.8 1.4) (end 2.2 2) (stroke (width 0.12) (type default)) (layer "F.SilkS"))
  (fp_line (start 2.8 1.4) (end 2.8 -2) (stroke (width 0.12) (type solid)) (layer "F.SilkS"))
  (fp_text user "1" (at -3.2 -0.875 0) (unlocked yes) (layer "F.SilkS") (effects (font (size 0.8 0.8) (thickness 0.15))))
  (pad "1" smd rect (at -1.75 -0.875) (size 1.6 0.85) (layers "F.Cu" "F.Mask" "F.Paste") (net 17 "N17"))
  (pad "2" smd rect (at -1.75 0.875) (size 1.6 0.85) (layers "F.Cu" "F.Mask" "F.Paste") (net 2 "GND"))
  (pad "3" smd rect (at 1.75 0.875) (size 1.6 0.85) (layers "F.Cu" "F.Mask" "F.Paste") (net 1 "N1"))
  (pad "4" smd rect (at 1.75 -0.875) (size 1.6 0.85) (layers "F.Cu" "F.Mask" "F.Paste") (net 4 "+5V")))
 (gr_rect (start 79.1 56.1) (end 139.9 119) (stroke (width 0.05) (type default)) (fill no) (layer "Edge.Cuts"))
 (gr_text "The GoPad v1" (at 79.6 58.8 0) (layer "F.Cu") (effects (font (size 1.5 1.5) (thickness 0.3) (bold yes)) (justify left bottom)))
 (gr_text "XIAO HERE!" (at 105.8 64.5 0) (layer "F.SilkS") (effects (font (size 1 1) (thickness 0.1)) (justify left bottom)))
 (segment (start 96.8 56.701) (end 126.5 56.701) (width 0.2) (layer "F.Cu") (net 4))
 (segment (start 126.5 56.9) (end 126.45 56.95) (width 0.2) (layer "F.Cu") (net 4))
 (segment (start 96.85 65.025) (end 96.85 56.751) (width 0.2) (layer "F.Cu") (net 4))
 (segment (start 96.85 56.751) (end 96.8 56.701) (width 0.2) (layer "F.Cu") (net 4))
 (segment (start 126.5 56.701) (end 126.5 56.9) (width 0.2) (layer "F.Cu") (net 4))
 (segment (start 126.45 56.95) (end 126.45 65.025) (width 0.2) (layer "F.Cu") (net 4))
 (segment (start 123 57.102) (end 123 57.3) (width 0.2) (layer "F.Cu") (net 1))
 (segment (start 123 57.3) (end 122.95 57.35) (width 0.2) (layer "F.Cu") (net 1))
 (segment (start 98 65.702) (end 98 57.2) (width 0.2) (layer "F.Cu") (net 1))
 (segment (start 98 57.2) (end 97.902 57.102) (width 0.2) (layer "F.Cu") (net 1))
 (segment (start 97.902 57.102) (end 123 57.102) (width 0.2) (layer "F.Cu") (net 1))
 (segment (start 96.85 66.775) (end 97.874 65.751) (width 0.2) (layer "F.Cu") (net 1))
 (segment (start 97.951 65.751) (end 98 65.702) (width 0.2) (layer "F.Cu") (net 1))
 (segment (start 122.95 57.35) (end 122.95 65.025) (width 0.2) (layer "F.Cu") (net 1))
 (segment (start 97.874 65.751) (end 97.951 65.751) (width 0.2) (layer "F.Cu") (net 1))
 (segment (start 103.657 67.7315) (end 125.4935 67.7315) (width 0.2) (layer "F.Cu") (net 3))
 (segment (start 102.18 69.2085) (end 103.657 67.7315) (width 0.2) (layer "F.Cu") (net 3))
 (segment (start 125.4935 67.7315) (end 126.45 66.775) (width 0.2) (layer "F.Cu") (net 3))
 (segment (start 93.35 66.95) (end 93.35 66.775) (width 0.2) (layer "F.Cu") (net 2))
 (segment (start 122.95 66.775) (end 123.676 66.049) (width 0.2) (layer "F.Cu") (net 2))
 (segment (start 121.6025 83.02625) (end 121.6025 92.55125) (width 0.2) (layer "F.Cu") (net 2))
 (segment (start 112.0775 102.07625) (end 93.0275 102.07625) (width 0.2) (layer "F.Cu") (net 2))
 (segment (start 121.849 65.674) (end 122.95 66.775) (width 0.2) (layer "F.Cu") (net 2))
 (segment (start 96.2025 69.9975) (end 96.3 69.9) (width 0.2) (layer "F.Cu") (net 2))
 (segment (start 128.9 66.4) (end 128.9 75.72875) (width 0.2) (layer "F.Cu") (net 2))
 (segment (start 128.9 75.72875) (end 121.6025 83.02625) (width 0.2) (layer "F.Cu") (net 2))
 (segment (start 121.6025 92.55125) (end 112.0775 102.07625) (width 0.2) (layer "F.Cu") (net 2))
 (segment (start 117.42 61.5885) (end 118.49763 61.5885) (width 0.2) (layer "F.Cu") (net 2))
 (segment (start 123.676 66.049) (end 128.549 66.049) (width 0.2) (layer "F.Cu") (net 2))
 (segment (start 112.0775 102.07625) (end 131.1275 102.07625) (width 0.2) (layer "F.Cu") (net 2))
 (segment (start 121.849 64.93987) (end 121.849 65.674) (width 0.2) (layer "F.Cu") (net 2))
 (segment (start 118.49763 61.5885) (end 121.849 64.93987) (width 0.2) (layer "F.Cu") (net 2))
 (segment (start 96.3 69.9) (end 93.35 66.95) (width 0.2) (layer "F.Cu") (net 2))
 (segment (start 96.2025 85.56625) (end 96.2025 69.9975) (width 0.2) (layer "F.Cu") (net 2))
 (segment (start 128.549 66.049) (end 128.9 66.4) (width 0.2) (layer "F.Cu") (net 2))
 (segment (start 96.2025 85.56625) (end 96.2025 98.90125) (width 0.2) (layer "B.Cu") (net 2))
 (segment (start 96.2025 98.90125) (end 93.0275 102.07625) (width 0.2) (layer "B.Cu") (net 2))
 (segment (start 111.29025 74.2885) (end 117.42 74.2885) (width 0.2) (layer "F.Cu") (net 5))
 (segment (start 102.5525 83.02625) (end 111.29025 74.2885) (width 0.2) (layer "F.Cu") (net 5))
 (segment (start 119.8 75.2) (end 116.9 78.1) (width 0.2) (layer "F.Cu") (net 12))
 (segment (start 117.42 71.7485) (end 118.49763 71.7485) (width 0.2) (layer "F.Cu") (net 12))
 (segment (start 116.9 83.91875) (end 115.2525 85.56625) (width 0.2) (layer "F.Cu") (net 12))
 (segment (start 118.49763 71.7485) (end 119.8 73.05087) (width 0.2) (layer "F.Cu") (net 12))
 (segment (start 119.8 73.05087) (end 119.8 75.2) (width 0.2) (layer "F.Cu") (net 12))
 (segment (start 116.9 78.1) (end 116.9 83.91875) (width 0.2) (layer "F.Cu") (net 12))
 (segment (start 97.8 86.993934) (end 86.6775 98.116434) (width 0.2) (layer "F.Cu") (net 13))
 (segment (start 86.6775 98.116434) (end 86.6775 104.61625) (width 0.2) (layer "F.Cu") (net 13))
 (segment (start 117.42 69.2085) (end 114.0915 69.2085) (width 0.2) (layer "F.Cu") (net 13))
 (segment (start 97.8 85.5) (end 97.8 86.993934) (width 0.2) (layer "F.Cu") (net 13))
 (segment (start 114.0915 69.2085) (end 97.8 85.5) (width 0.2) (layer "F.Cu") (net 13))
 (segment (start 106.827499 103.516251) (end 106.827499 77.261001) (width 0.2) (layer "B.Cu") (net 14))
 (segment (start 106.827499 77.261001) (end 117.42 66.6685) (width 0.2) (layer "B.Cu") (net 14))
 (segment (start 105.7275 104.61625) (end 106.827499 103.516251) (width 0.2) (layer "B.Cu") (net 14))
 (segment (start 120.2015 66.91) (end 120.2015 85.920434) (width 0.2) (layer "B.Cu") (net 15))
 (segment (start 120.2015 85.920434) (end 124.7775 90.496434) (width 0.2) (layer "B.Cu") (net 15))
 (segment (start 117.42 64.1285) (end 120.2015 66.91) (width 0.2) (layer "B.Cu") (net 15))
 (segment (start 124.7775 90.496434) (end 124.7775 104.61625) (width 0.2) (layer "B.Cu") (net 15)))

